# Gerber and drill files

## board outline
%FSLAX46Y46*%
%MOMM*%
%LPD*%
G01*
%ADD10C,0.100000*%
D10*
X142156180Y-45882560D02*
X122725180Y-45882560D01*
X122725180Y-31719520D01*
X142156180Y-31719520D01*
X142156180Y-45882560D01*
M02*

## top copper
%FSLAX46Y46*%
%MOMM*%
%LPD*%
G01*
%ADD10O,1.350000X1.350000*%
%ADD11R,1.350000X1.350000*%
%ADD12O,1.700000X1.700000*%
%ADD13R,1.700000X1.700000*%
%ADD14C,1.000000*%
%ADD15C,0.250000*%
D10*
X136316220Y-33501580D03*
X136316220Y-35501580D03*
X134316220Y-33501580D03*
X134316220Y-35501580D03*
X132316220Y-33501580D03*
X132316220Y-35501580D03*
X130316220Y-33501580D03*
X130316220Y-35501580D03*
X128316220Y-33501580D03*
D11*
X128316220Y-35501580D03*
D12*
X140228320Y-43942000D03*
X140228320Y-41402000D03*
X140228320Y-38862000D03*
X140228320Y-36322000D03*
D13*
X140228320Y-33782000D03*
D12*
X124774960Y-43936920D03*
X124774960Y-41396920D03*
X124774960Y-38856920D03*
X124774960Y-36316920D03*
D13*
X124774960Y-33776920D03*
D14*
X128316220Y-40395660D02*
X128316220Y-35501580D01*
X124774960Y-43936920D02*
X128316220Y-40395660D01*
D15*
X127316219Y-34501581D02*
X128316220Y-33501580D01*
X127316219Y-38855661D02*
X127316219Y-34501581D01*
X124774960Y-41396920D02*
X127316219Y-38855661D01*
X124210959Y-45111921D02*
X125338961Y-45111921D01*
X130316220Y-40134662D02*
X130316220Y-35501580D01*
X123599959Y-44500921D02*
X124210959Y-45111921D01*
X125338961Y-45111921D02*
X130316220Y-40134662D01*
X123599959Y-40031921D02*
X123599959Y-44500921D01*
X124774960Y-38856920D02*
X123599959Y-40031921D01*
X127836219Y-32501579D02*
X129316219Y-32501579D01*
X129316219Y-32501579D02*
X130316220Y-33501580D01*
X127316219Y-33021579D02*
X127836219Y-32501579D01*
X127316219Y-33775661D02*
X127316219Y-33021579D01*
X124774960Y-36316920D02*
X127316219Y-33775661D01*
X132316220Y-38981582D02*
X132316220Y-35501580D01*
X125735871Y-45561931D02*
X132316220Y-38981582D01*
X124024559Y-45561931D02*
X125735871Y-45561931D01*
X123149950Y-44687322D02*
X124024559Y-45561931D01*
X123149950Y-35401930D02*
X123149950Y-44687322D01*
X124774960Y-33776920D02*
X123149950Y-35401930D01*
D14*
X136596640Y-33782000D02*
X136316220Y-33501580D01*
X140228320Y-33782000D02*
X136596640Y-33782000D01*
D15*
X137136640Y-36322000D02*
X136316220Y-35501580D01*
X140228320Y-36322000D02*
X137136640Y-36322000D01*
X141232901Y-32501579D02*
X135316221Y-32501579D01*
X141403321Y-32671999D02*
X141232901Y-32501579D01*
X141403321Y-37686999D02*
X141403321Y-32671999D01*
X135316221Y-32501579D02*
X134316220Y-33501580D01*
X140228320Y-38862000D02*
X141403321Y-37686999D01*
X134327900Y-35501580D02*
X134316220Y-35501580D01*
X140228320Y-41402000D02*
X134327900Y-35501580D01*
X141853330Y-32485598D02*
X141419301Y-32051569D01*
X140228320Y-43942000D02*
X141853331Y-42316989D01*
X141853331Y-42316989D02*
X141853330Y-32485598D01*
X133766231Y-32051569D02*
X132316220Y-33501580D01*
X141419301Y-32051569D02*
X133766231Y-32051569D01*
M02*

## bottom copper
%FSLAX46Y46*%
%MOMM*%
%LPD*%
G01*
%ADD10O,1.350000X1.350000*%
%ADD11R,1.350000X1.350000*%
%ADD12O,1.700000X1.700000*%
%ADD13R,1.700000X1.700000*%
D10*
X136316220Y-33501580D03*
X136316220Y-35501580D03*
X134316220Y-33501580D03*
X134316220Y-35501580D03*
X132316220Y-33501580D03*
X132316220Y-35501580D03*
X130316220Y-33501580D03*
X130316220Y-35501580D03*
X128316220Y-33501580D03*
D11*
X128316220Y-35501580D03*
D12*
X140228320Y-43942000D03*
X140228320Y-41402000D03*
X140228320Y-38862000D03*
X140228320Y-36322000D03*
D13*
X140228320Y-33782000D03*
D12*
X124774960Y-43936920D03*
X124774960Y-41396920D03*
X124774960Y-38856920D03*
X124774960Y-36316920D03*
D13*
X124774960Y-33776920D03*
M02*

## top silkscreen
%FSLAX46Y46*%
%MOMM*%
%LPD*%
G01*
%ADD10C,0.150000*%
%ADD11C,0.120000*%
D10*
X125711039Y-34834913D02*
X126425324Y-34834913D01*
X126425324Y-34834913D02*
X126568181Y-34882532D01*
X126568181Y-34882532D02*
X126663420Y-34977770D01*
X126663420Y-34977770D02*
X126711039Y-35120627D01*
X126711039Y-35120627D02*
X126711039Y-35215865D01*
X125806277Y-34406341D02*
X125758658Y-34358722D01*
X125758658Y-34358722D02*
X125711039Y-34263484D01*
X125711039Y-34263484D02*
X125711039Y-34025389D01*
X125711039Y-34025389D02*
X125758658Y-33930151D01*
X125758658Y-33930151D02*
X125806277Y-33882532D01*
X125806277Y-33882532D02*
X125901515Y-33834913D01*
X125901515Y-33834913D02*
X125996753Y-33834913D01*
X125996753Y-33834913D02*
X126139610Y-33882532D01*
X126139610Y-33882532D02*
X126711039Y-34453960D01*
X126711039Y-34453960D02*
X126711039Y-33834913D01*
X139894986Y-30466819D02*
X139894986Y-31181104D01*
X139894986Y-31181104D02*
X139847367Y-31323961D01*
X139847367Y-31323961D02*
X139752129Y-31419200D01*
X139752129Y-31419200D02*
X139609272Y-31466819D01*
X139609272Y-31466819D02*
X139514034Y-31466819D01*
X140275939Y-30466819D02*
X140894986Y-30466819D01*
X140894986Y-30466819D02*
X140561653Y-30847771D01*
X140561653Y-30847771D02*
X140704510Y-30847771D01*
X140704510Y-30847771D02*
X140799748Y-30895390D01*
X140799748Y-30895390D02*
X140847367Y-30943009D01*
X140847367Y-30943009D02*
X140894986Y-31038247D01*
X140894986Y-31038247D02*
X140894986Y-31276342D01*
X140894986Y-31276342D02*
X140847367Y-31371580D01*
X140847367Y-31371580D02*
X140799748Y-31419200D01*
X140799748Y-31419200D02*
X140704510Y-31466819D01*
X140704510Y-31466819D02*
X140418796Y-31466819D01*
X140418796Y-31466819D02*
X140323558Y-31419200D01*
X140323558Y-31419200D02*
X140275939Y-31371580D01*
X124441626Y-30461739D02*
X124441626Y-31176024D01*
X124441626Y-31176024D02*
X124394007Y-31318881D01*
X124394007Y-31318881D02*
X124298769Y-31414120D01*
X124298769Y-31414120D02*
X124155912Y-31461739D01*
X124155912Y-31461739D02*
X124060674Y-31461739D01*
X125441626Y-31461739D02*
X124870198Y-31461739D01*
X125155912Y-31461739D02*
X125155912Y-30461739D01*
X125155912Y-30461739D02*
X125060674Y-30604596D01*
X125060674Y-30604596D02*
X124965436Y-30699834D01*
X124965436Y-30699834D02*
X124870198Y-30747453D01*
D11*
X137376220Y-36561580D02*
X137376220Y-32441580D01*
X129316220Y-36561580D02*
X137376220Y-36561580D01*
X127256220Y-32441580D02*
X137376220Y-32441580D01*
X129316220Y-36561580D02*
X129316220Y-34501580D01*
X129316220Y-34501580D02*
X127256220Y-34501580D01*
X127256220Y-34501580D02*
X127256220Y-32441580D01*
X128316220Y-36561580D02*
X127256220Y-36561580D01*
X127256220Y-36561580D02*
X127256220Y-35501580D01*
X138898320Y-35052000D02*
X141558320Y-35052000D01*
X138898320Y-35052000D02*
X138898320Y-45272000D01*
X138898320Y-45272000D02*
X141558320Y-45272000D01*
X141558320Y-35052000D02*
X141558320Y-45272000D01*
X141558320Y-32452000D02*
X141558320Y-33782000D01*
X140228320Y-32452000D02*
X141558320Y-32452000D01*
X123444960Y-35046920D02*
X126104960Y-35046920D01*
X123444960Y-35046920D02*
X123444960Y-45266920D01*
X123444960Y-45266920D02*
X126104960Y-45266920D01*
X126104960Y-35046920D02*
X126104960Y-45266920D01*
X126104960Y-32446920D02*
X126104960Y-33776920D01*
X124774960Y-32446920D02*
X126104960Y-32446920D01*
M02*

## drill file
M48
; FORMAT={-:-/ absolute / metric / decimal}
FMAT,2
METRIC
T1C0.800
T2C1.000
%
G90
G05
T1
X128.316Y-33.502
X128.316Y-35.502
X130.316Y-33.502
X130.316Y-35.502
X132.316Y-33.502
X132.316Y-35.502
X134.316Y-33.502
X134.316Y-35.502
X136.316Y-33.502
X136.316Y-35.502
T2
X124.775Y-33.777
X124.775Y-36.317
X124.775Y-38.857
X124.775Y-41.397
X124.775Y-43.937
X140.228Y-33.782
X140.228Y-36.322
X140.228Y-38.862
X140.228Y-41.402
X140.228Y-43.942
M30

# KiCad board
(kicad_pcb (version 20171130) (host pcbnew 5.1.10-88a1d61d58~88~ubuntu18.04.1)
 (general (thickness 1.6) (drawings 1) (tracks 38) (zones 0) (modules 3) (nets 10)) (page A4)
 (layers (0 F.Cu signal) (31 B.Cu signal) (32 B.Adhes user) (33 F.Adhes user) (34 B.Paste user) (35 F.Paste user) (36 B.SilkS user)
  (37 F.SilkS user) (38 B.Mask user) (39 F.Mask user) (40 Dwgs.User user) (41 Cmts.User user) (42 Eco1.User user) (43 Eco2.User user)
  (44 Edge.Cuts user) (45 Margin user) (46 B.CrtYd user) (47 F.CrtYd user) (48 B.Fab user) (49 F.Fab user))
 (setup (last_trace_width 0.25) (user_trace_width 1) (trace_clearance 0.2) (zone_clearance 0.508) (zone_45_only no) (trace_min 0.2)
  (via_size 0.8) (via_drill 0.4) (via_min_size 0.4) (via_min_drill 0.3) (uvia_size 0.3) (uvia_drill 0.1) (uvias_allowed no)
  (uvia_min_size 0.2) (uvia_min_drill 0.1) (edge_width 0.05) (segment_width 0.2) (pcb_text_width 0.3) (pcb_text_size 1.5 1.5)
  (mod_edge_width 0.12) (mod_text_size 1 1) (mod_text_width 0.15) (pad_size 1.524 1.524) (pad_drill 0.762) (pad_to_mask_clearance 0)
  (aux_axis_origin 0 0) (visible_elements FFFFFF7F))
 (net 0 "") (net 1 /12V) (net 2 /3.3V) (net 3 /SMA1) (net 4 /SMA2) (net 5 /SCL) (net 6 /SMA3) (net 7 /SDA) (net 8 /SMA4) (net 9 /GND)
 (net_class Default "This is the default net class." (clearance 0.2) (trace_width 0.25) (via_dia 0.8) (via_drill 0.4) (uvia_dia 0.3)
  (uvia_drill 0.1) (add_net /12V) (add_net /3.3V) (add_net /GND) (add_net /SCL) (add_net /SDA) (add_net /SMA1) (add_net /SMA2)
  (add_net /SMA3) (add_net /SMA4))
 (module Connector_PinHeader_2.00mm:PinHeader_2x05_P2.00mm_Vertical (layer F.Cu) (at 128.31622 35.50158 90)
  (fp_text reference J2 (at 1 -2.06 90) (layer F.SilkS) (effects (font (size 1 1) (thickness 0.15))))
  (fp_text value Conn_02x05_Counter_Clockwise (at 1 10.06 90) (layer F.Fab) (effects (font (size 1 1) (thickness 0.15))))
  (fp_line (start -1.06 9.06) (end 3.06 9.06) (layer F.SilkS) (width 0.12))
  (fp_line (start -1.06 1) (end -1.06 9.06) (layer F.SilkS) (width 0.12))
  (fp_line (start 3.06 -1.06) (end 3.06 9.06) (layer F.SilkS) (width 0.12))
  (fp_line (start -1.06 1) (end 1 1) (layer F.SilkS) (width 0.12))
  (fp_line (start 1 1) (end 1 -1.06) (layer F.SilkS) (width 0.12))
  (fp_line (start 1 -1.06) (end 3.06 -1.06) (layer F.SilkS) (width 0.12))
  (fp_line (start -1.06 0) (end -1.06 -1.06) (layer F.SilkS) (width 0.12))
  (fp_line (start -1.06 -1.06) (end 0 -1.06) (layer F.SilkS) (width 0.12))
  (pad 10 thru_hole oval (at 2 8 90) (size 1.35 1.35) (drill 0.8) (layers *.Cu *.Mask) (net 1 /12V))
  (pad 9 thru_hole oval (at 0 8 90) (size 1.35 1.35) (drill 0.8) (layers *.Cu *.Mask) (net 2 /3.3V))
  (pad 8 thru_hole oval (at 2 6 90) (size 1.35 1.35) (drill 0.8) (layers *.Cu *.Mask) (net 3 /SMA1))
  (pad 7 thru_hole oval (at 0 6 90) (size 1.35 1.35) (drill 0.8) (layers *.Cu *.Mask) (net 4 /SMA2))
  (pad 6 thru_hole oval (at 2 4 90) (size 1.35 1.35) (drill 0.8) (layers *.Cu *.Mask) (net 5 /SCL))
  (pad 5 thru_hole oval (at 0 4 90) (size 1.35 1.35) (drill 0.8) (layers *.Cu *.Mask) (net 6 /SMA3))
  (pad 4 thru_hole oval (at 2 2 90) (size 1.35 1.35) (drill 0.8) (layers *.Cu *.Mask) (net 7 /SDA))
  (pad 3 thru_hole oval (at 0 2 90) (size 1.35 1.35) (drill 0.8) (layers *.Cu *.Mask) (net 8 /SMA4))
  (pad 2 thru_hole oval (at 2 0 90) (size 1.35 1.35) (drill 0.8) (layers *.Cu *.Mask) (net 8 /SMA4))
  (pad 1 thru_hole rect (at 0 0 90) (size 1.35 1.35) (drill 0.8) (layers *.Cu *.Mask) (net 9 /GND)))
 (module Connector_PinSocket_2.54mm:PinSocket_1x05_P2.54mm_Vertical (layer F.Cu) (at 140.22832 33.782)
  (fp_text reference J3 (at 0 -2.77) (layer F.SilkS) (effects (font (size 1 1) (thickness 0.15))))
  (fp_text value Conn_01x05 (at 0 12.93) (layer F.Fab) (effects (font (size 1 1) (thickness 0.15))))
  (fp_line (start -1.33 1.27) (end 1.33 1.27) (layer F.SilkS) (width 0.12))
  (fp_line (start -1.33 1.27) (end -1.33 11.49) (layer F.SilkS) (width 0.12))
  (fp_line (start -1.33 11.49) (end 1.33 11.49) (layer F.SilkS) (width 0.12))
  (fp_line (start 1.33 1.27) (end 1.33 11.49) (layer F.SilkS) (width 0.12))
  (fp_line (start 1.33 -1.33) (end 1.33 0) (layer F.SilkS) (width 0.12))
  (fp_line (start 0 -1.33) (end 1.33 -1.33) (layer F.SilkS) (width 0.12))
  (pad 5 thru_hole oval (at 0 10.16) (size 1.7 1.7) (drill 1) (layers *.Cu *.Mask) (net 5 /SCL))
  (pad 4 thru_hole oval (at 0 7.62) (size 1.7 1.7) (drill 1) (layers *.Cu *.Mask) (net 4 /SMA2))
  (pad 3 thru_hole oval (at 0 5.08) (size 1.7 1.7) (drill 1) (layers *.Cu *.Mask) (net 3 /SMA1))
  (pad 2 thru_hole oval (at 0 2.54) (size 1.7 1.7) (drill 1) (layers *.Cu *.Mask) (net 2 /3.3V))
  (pad 1 thru_hole rect (at 0 0) (size 1.7 1.7) (drill 1) (layers *.Cu *.Mask) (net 1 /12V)))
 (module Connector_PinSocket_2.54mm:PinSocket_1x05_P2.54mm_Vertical (layer F.Cu) (at 124.77496 33.77692)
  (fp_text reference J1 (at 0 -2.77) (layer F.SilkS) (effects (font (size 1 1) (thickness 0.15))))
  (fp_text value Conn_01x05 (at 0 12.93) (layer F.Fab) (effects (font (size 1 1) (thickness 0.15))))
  (fp_line (start -1.33 1.27) (end 1.33 1.27) (layer F.SilkS) (width 0.12))
  (fp_line (start -1.33 1.27) (end -1.33 11.49) (layer F.SilkS) (width 0.12))
  (fp_line (start -1.33 11.49) (end 1.33 11.49) (layer F.SilkS) (width 0.12))
  (fp_line (start 1.33 1.27) (end 1.33 11.49) (layer F.SilkS) (width 0.12))
  (fp_line (start 1.33 -1.33) (end 1.33 0) (layer F.SilkS) (width 0.12))
  (fp_line (start 0 -1.33) (end 1.33 -1.33) (layer F.SilkS) (width 0.12))
  (pad 5 thru_hole oval (at 0 10.16) (size 1.7 1.7) (drill 1) (layers *.Cu *.Mask) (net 9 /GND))
  (pad 4 thru_hole oval (at 0 7.62) (size 1.7 1.7) (drill 1) (layers *.Cu *.Mask) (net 8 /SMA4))
  (pad 3 thru_hole oval (at 0 5.08) (size 1.7 1.7) (drill 1) (layers *.Cu *.Mask) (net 8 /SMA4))
  (pad 2 thru_hole oval (at 0 2.54) (size 1.7 1.7) (drill 1) (layers *.Cu *.Mask) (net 7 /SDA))
  (pad 1 thru_hole rect (at 0 0) (size 1.7 1.7) (drill 1) (layers *.Cu *.Mask) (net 6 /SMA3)))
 (gr_poly
  (pts (xy 142.15618 45.88256) (xy 122.72518 45.88256) (xy 122.72518 31.71952) (xy 142.15618 31.71952)) (layer Edge.Cuts) (width 0.1))
 (segment (start 128.31622 40.39566) (end 128.31622 35.50158) (width 1) (layer F.Cu) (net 9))
 (segment (start 124.77496 43.93692) (end 128.31622 40.39566) (width 1) (layer F.Cu) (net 9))
 (segment (start 127.316219 34.501581) (end 128.31622 33.50158) (width 0.25) (layer F.Cu) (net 8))
 (segment (start 127.316219 38.855661) (end 127.316219 34.501581) (width 0.25) (layer F.Cu) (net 8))
 (segment (start 124.77496 41.39692) (end 127.316219 38.855661) (width 0.25) (layer F.Cu) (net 8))
 (segment (start 124.210959 45.111921) (end 125.338961 45.111921) (width 0.25) (layer F.Cu) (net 8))
 (segment (start 130.31622 40.134662) (end 130.31622 35.50158) (width 0.25) (layer F.Cu) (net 8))
 (segment (start 123.599959 44.500921) (end 124.210959 45.111921) (width 0.25) (layer F.Cu) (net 8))
 (segment (start 125.338961 45.111921) (end 130.31622 40.134662) (width 0.25) (layer F.Cu) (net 8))
 (segment (start 123.599959 40.031921) (end 123.599959 44.500921) (width 0.25) (layer F.Cu) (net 8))
 (segment (start 124.77496 38.85692) (end 123.599959 40.031921) (width 0.25) (layer F.Cu) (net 8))
 (segment (start 127.836219 32.501579) (end 129.316219 32.501579) (width 0.25) (layer F.Cu) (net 7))
 (segment (start 129.316219 32.501579) (end 130.31622 33.50158) (width 0.25) (layer F.Cu) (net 7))
 (segment (start 127.316219 33.021579) (end 127.836219 32.501579) (width 0.25) (layer F.Cu) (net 7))
 (segment (start 127.316219 33.775661) (end 127.316219 33.021579) (width 0.25) (layer F.Cu) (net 7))
 (segment (start 124.77496 36.31692) (end 127.316219 33.775661) (width 0.25) (layer F.Cu) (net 7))
 (segment (start 132.31622 38.981582) (end 132.31622 35.50158) (width 0.25) (layer F.Cu) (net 6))
 (segment (start 125.735871 45.561931) (end 132.31622 38.981582) (width 0.25) (layer F.Cu) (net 6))
 (segment (start 124.024559 45.561931) (end 125.735871 45.561931) (width 0.25) (layer F.Cu) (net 6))
 (segment (start 123.14995 44.687322) (end 124.024559 45.561931) (width 0.25) (layer F.Cu) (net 6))
 (segment (start 123.14995 35.40193) (end 123.14995 44.687322) (width 0.25) (layer F.Cu) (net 6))
 (segment (start 124.77496 33.77692) (end 123.14995 35.40193) (width 0.25) (layer F.Cu) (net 6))
 (segment (start 136.59664 33.782) (end 136.31622 33.50158) (width 1) (layer F.Cu) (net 1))
 (segment (start 140.22832 33.782) (end 136.59664 33.782) (width 1) (layer F.Cu) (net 1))
 (segment (start 137.13664 36.322) (end 136.31622 35.50158) (width 0.25) (layer F.Cu) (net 2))
 (segment (start 140.22832 36.322) (end 137.13664 36.322) (width 0.25) (layer F.Cu) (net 2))
 (segment (start 141.232901 32.501579) (end 135.316221 32.501579) (width 0.25) (layer F.Cu) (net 3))
 (segment (start 141.403321 32.671999) (end 141.232901 32.501579) (width 0.25) (layer F.Cu) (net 3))
 (segment (start 141.403321 37.686999) (end 141.403321 32.671999) (width 0.25) (layer F.Cu) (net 3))
 (segment (start 135.316221 32.501579) (end 134.31622 33.50158) (width 0.25) (layer F.Cu) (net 3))
 (segment (start 140.22832 38.862) (end 141.403321 37.686999) (width 0.25) (layer F.Cu) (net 3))
 (segment (start 134.3279 35.50158) (end 134.31622 35.50158) (width 0.25) (layer F.Cu) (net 4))
 (segment (start 140.22832 41.402) (end 134.3279 35.50158) (width 0.25) (layer F.Cu) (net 4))
 (segment (start 141.85333 32.485598) (end 141.419301 32.051569) (width 0.25) (layer F.Cu) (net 5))
 (segment (start 140.22832 43.942) (end 141.853331 42.316989) (width 0.25) (layer F.Cu) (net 5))
 (segment (start 141.853331 42.316989) (end 141.85333 32.485598) (width 0.25) (layer F.Cu) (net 5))
 (segment (start 133.766231 32.051569) (end 132.31622 33.50158) (width 0.25) (layer F.Cu) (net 5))
 (segment (start 141.419301 32.051569) (end 133.766231 32.051569) (width 0.25) (layer F.Cu) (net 5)))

